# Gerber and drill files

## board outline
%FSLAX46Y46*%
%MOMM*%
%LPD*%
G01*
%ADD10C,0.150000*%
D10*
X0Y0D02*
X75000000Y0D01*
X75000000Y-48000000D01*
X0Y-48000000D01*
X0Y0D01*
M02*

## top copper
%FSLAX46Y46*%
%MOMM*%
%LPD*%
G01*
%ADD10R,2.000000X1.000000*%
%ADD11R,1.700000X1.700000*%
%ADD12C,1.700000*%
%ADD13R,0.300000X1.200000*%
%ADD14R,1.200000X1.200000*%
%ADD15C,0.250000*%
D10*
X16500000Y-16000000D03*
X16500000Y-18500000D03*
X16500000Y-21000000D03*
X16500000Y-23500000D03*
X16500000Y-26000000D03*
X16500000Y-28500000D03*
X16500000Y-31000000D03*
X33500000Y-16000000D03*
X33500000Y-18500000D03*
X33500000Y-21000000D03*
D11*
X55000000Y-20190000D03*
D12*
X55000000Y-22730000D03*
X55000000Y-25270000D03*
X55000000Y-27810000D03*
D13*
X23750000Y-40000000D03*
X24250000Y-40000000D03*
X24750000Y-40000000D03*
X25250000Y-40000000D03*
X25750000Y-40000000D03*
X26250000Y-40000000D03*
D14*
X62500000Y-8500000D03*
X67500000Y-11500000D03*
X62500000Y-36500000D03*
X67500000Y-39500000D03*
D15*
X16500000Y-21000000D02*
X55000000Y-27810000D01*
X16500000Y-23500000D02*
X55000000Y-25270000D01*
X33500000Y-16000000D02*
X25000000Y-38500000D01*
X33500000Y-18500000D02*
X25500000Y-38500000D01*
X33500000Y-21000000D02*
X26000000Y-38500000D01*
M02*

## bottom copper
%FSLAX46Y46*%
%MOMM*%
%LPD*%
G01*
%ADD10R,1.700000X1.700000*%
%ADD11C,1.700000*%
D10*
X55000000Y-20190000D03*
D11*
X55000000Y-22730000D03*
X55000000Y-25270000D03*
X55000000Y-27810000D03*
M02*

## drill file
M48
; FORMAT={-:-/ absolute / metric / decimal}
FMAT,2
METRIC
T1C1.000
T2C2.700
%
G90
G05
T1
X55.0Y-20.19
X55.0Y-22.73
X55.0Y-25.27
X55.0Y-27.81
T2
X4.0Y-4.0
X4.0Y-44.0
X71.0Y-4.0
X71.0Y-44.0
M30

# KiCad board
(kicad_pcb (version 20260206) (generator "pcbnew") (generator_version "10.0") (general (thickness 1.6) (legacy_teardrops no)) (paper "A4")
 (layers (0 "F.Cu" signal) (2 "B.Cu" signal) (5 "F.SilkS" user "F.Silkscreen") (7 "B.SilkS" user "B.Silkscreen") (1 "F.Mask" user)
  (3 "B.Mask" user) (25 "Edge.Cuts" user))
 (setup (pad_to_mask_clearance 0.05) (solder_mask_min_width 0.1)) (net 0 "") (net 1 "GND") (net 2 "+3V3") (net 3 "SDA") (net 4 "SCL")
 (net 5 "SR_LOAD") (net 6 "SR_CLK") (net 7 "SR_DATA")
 (gr_rect (start 0 0) (end 75.0 48.0) (stroke (width 0.15) (type solid)) (fill none) (layer "Edge.Cuts"))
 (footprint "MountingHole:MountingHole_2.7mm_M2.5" (layer "F.Cu") (at 4 4)
  (pad "1" np_thru_hole circle (at 0 0) (size 2.7 2.7) (drill 2.7) (layers "*.Cu" "*.Mask")))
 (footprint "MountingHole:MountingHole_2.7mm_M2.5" (layer "F.Cu") (at 71.0 4)
  (pad "1" np_thru_hole circle (at 0 0) (size 2.7 2.7) (drill 2.7) (layers "*.Cu" "*.Mask")))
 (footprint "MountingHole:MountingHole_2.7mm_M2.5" (layer "F.Cu") (at 4 44.0)
  (pad "1" np_thru_hole circle (at 0 0) (size 2.7 2.7) (drill 2.7) (layers "*.Cu" "*.Mask")))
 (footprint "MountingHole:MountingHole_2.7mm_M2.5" (layer "F.Cu") (at 71.0 44.0)
  (pad "1" np_thru_hole circle (at 0 0) (size 2.7 2.7) (drill 2.7) (layers "*.Cu" "*.Mask")))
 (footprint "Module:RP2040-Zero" (layer "F.Cu") (at 25.0 24.0)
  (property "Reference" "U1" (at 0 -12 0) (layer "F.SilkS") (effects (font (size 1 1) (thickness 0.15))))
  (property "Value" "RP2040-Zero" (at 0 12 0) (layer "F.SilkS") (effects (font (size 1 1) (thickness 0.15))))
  (pad "1" smd rect (at -8.5 -8) (size 2.0 1.0) (layers "F.Cu" "F.Paste" "F.Mask") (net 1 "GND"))
  (pad "2" smd rect (at -8.5 -5.5) (size 2.0 1.0) (layers "F.Cu" "F.Paste" "F.Mask") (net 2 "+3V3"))
  (pad "3" smd rect (at -8.5 -3) (size 2.0 1.0) (layers "F.Cu" "F.Paste" "F.Mask") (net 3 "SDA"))
  (pad "4" smd rect (at -8.5 -0.5) (size 2.0 1.0) (layers "F.Cu" "F.Paste" "F.Mask") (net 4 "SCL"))
  (pad "5" smd rect (at -8.5 2) (size 2.0 1.0) (layers "F.Cu" "F.Paste" "F.Mask"))
  (pad "6" smd rect (at -8.5 4.5) (size 2.0 1.0) (layers "F.Cu" "F.Paste" "F.Mask"))
  (pad "7" smd rect (at -8.5 7) (size 2.0 1.0) (layers "F.Cu" "F.Paste" "F.Mask"))
  (pad "8" smd rect (at 8.5 -8) (size 2.0 1.0) (layers "F.Cu" "F.Paste" "F.Mask") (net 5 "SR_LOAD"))
  (pad "9" smd rect (at 8.5 -5.5) (size 2.0 1.0) (layers "F.Cu" "F.Paste" "F.Mask") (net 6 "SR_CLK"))
  (pad "10" smd rect (at 8.5 -3) (size 2.0 1.0) (layers "F.Cu" "F.Paste" "F.Mask") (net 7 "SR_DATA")))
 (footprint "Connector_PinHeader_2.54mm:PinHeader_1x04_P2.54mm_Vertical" (layer "F.Cu") (at 55.0 24.0)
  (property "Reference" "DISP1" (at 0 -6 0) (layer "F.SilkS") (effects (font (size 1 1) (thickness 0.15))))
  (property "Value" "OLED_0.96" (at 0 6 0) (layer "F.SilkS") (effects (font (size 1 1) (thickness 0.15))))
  (pad "1" thru_hole rect (at 0 -3.81) (size 1.7 1.7) (drill 1.0) (layers "*.Cu" "*.Mask") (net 1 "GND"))
  (pad "2" thru_hole circle (at 0 -1.27) (size 1.7 1.7) (drill 1.0) (layers "*.Cu" "*.Mask") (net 2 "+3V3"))
  (pad "3" thru_hole circle (at 0 1.27) (size 1.7 1.7) (drill 1.0) (layers "*.Cu" "*.Mask") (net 4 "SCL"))
  (pad "4" thru_hole circle (at 0 3.81) (size 1.7 1.7) (drill 1.0) (layers "*.Cu" "*.Mask") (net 3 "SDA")))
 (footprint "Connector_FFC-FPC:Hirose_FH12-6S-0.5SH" (layer "F.Cu") (at 25 40)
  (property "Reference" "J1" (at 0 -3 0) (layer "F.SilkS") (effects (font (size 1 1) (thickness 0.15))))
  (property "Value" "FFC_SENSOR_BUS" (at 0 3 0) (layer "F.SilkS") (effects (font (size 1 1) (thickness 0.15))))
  (pad "1" smd rect (at -1.25 0) (size 0.3 1.2) (layers "F.Cu" "F.Paste" "F.Mask") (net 1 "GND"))
  (pad "2" smd rect (at -0.75 0) (size 0.3 1.2) (layers "F.Cu" "F.Paste" "F.Mask") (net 2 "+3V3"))
  (pad "3" smd rect (at -0.25 0) (size 0.3 1.2) (layers "F.Cu" "F.Paste" "F.Mask") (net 5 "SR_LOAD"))
  (pad "4" smd rect (at 0.25 0) (size 0.3 1.2) (layers "F.Cu" "F.Paste" "F.Mask") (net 6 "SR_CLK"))
  (pad "5" smd rect (at 0.75 0) (size 0.3 1.2) (layers "F.Cu" "F.Paste" "F.Mask") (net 7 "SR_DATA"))
  (pad "6" smd rect (at 1.25 0) (size 0.3 1.2) (layers "F.Cu" "F.Paste" "F.Mask") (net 1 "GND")))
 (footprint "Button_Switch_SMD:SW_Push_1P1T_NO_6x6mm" (layer "F.Cu") (at 65 10)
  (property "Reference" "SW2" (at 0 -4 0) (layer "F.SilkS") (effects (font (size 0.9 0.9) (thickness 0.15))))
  (pad "1" smd rect (at -2.5 -1.5) (size 1.2 1.2) (layers "F.Cu" "F.Paste" "F.Mask") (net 1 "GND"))
  (pad "2" smd rect (at 2.5 1.5) (size 1.2 1.2) (layers "F.Cu" "F.Paste" "F.Mask")))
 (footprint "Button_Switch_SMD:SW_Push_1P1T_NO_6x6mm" (layer "F.Cu") (at 65 38)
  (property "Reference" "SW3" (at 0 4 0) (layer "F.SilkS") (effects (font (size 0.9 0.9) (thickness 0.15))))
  (pad "1" smd rect (at -2.5 -1.5) (size 1.2 1.2) (layers "F.Cu" "F.Paste" "F.Mask") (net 1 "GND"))
  (pad "2" smd rect (at 2.5 1.5) (size 1.2 1.2) (layers "F.Cu" "F.Paste" "F.Mask")))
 (segment (start 16.5 21.0) (end 55.0 27.81) (width 0.25) (layer "F.Cu") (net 3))
 (segment (start 16.5 23.5) (end 55.0 25.27) (width 0.25) (layer "F.Cu") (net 4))
 (segment (start 33.5 16.0) (end 25 38.5) (width 0.25) (layer "F.Cu") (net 5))
 (segment (start 33.5 18.5) (end 25.5 38.5) (width 0.25) (layer "F.Cu") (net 6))
 (segment (start 33.5 21.0) (end 26 38.5) (width 0.25) (layer "F.Cu") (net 7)))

